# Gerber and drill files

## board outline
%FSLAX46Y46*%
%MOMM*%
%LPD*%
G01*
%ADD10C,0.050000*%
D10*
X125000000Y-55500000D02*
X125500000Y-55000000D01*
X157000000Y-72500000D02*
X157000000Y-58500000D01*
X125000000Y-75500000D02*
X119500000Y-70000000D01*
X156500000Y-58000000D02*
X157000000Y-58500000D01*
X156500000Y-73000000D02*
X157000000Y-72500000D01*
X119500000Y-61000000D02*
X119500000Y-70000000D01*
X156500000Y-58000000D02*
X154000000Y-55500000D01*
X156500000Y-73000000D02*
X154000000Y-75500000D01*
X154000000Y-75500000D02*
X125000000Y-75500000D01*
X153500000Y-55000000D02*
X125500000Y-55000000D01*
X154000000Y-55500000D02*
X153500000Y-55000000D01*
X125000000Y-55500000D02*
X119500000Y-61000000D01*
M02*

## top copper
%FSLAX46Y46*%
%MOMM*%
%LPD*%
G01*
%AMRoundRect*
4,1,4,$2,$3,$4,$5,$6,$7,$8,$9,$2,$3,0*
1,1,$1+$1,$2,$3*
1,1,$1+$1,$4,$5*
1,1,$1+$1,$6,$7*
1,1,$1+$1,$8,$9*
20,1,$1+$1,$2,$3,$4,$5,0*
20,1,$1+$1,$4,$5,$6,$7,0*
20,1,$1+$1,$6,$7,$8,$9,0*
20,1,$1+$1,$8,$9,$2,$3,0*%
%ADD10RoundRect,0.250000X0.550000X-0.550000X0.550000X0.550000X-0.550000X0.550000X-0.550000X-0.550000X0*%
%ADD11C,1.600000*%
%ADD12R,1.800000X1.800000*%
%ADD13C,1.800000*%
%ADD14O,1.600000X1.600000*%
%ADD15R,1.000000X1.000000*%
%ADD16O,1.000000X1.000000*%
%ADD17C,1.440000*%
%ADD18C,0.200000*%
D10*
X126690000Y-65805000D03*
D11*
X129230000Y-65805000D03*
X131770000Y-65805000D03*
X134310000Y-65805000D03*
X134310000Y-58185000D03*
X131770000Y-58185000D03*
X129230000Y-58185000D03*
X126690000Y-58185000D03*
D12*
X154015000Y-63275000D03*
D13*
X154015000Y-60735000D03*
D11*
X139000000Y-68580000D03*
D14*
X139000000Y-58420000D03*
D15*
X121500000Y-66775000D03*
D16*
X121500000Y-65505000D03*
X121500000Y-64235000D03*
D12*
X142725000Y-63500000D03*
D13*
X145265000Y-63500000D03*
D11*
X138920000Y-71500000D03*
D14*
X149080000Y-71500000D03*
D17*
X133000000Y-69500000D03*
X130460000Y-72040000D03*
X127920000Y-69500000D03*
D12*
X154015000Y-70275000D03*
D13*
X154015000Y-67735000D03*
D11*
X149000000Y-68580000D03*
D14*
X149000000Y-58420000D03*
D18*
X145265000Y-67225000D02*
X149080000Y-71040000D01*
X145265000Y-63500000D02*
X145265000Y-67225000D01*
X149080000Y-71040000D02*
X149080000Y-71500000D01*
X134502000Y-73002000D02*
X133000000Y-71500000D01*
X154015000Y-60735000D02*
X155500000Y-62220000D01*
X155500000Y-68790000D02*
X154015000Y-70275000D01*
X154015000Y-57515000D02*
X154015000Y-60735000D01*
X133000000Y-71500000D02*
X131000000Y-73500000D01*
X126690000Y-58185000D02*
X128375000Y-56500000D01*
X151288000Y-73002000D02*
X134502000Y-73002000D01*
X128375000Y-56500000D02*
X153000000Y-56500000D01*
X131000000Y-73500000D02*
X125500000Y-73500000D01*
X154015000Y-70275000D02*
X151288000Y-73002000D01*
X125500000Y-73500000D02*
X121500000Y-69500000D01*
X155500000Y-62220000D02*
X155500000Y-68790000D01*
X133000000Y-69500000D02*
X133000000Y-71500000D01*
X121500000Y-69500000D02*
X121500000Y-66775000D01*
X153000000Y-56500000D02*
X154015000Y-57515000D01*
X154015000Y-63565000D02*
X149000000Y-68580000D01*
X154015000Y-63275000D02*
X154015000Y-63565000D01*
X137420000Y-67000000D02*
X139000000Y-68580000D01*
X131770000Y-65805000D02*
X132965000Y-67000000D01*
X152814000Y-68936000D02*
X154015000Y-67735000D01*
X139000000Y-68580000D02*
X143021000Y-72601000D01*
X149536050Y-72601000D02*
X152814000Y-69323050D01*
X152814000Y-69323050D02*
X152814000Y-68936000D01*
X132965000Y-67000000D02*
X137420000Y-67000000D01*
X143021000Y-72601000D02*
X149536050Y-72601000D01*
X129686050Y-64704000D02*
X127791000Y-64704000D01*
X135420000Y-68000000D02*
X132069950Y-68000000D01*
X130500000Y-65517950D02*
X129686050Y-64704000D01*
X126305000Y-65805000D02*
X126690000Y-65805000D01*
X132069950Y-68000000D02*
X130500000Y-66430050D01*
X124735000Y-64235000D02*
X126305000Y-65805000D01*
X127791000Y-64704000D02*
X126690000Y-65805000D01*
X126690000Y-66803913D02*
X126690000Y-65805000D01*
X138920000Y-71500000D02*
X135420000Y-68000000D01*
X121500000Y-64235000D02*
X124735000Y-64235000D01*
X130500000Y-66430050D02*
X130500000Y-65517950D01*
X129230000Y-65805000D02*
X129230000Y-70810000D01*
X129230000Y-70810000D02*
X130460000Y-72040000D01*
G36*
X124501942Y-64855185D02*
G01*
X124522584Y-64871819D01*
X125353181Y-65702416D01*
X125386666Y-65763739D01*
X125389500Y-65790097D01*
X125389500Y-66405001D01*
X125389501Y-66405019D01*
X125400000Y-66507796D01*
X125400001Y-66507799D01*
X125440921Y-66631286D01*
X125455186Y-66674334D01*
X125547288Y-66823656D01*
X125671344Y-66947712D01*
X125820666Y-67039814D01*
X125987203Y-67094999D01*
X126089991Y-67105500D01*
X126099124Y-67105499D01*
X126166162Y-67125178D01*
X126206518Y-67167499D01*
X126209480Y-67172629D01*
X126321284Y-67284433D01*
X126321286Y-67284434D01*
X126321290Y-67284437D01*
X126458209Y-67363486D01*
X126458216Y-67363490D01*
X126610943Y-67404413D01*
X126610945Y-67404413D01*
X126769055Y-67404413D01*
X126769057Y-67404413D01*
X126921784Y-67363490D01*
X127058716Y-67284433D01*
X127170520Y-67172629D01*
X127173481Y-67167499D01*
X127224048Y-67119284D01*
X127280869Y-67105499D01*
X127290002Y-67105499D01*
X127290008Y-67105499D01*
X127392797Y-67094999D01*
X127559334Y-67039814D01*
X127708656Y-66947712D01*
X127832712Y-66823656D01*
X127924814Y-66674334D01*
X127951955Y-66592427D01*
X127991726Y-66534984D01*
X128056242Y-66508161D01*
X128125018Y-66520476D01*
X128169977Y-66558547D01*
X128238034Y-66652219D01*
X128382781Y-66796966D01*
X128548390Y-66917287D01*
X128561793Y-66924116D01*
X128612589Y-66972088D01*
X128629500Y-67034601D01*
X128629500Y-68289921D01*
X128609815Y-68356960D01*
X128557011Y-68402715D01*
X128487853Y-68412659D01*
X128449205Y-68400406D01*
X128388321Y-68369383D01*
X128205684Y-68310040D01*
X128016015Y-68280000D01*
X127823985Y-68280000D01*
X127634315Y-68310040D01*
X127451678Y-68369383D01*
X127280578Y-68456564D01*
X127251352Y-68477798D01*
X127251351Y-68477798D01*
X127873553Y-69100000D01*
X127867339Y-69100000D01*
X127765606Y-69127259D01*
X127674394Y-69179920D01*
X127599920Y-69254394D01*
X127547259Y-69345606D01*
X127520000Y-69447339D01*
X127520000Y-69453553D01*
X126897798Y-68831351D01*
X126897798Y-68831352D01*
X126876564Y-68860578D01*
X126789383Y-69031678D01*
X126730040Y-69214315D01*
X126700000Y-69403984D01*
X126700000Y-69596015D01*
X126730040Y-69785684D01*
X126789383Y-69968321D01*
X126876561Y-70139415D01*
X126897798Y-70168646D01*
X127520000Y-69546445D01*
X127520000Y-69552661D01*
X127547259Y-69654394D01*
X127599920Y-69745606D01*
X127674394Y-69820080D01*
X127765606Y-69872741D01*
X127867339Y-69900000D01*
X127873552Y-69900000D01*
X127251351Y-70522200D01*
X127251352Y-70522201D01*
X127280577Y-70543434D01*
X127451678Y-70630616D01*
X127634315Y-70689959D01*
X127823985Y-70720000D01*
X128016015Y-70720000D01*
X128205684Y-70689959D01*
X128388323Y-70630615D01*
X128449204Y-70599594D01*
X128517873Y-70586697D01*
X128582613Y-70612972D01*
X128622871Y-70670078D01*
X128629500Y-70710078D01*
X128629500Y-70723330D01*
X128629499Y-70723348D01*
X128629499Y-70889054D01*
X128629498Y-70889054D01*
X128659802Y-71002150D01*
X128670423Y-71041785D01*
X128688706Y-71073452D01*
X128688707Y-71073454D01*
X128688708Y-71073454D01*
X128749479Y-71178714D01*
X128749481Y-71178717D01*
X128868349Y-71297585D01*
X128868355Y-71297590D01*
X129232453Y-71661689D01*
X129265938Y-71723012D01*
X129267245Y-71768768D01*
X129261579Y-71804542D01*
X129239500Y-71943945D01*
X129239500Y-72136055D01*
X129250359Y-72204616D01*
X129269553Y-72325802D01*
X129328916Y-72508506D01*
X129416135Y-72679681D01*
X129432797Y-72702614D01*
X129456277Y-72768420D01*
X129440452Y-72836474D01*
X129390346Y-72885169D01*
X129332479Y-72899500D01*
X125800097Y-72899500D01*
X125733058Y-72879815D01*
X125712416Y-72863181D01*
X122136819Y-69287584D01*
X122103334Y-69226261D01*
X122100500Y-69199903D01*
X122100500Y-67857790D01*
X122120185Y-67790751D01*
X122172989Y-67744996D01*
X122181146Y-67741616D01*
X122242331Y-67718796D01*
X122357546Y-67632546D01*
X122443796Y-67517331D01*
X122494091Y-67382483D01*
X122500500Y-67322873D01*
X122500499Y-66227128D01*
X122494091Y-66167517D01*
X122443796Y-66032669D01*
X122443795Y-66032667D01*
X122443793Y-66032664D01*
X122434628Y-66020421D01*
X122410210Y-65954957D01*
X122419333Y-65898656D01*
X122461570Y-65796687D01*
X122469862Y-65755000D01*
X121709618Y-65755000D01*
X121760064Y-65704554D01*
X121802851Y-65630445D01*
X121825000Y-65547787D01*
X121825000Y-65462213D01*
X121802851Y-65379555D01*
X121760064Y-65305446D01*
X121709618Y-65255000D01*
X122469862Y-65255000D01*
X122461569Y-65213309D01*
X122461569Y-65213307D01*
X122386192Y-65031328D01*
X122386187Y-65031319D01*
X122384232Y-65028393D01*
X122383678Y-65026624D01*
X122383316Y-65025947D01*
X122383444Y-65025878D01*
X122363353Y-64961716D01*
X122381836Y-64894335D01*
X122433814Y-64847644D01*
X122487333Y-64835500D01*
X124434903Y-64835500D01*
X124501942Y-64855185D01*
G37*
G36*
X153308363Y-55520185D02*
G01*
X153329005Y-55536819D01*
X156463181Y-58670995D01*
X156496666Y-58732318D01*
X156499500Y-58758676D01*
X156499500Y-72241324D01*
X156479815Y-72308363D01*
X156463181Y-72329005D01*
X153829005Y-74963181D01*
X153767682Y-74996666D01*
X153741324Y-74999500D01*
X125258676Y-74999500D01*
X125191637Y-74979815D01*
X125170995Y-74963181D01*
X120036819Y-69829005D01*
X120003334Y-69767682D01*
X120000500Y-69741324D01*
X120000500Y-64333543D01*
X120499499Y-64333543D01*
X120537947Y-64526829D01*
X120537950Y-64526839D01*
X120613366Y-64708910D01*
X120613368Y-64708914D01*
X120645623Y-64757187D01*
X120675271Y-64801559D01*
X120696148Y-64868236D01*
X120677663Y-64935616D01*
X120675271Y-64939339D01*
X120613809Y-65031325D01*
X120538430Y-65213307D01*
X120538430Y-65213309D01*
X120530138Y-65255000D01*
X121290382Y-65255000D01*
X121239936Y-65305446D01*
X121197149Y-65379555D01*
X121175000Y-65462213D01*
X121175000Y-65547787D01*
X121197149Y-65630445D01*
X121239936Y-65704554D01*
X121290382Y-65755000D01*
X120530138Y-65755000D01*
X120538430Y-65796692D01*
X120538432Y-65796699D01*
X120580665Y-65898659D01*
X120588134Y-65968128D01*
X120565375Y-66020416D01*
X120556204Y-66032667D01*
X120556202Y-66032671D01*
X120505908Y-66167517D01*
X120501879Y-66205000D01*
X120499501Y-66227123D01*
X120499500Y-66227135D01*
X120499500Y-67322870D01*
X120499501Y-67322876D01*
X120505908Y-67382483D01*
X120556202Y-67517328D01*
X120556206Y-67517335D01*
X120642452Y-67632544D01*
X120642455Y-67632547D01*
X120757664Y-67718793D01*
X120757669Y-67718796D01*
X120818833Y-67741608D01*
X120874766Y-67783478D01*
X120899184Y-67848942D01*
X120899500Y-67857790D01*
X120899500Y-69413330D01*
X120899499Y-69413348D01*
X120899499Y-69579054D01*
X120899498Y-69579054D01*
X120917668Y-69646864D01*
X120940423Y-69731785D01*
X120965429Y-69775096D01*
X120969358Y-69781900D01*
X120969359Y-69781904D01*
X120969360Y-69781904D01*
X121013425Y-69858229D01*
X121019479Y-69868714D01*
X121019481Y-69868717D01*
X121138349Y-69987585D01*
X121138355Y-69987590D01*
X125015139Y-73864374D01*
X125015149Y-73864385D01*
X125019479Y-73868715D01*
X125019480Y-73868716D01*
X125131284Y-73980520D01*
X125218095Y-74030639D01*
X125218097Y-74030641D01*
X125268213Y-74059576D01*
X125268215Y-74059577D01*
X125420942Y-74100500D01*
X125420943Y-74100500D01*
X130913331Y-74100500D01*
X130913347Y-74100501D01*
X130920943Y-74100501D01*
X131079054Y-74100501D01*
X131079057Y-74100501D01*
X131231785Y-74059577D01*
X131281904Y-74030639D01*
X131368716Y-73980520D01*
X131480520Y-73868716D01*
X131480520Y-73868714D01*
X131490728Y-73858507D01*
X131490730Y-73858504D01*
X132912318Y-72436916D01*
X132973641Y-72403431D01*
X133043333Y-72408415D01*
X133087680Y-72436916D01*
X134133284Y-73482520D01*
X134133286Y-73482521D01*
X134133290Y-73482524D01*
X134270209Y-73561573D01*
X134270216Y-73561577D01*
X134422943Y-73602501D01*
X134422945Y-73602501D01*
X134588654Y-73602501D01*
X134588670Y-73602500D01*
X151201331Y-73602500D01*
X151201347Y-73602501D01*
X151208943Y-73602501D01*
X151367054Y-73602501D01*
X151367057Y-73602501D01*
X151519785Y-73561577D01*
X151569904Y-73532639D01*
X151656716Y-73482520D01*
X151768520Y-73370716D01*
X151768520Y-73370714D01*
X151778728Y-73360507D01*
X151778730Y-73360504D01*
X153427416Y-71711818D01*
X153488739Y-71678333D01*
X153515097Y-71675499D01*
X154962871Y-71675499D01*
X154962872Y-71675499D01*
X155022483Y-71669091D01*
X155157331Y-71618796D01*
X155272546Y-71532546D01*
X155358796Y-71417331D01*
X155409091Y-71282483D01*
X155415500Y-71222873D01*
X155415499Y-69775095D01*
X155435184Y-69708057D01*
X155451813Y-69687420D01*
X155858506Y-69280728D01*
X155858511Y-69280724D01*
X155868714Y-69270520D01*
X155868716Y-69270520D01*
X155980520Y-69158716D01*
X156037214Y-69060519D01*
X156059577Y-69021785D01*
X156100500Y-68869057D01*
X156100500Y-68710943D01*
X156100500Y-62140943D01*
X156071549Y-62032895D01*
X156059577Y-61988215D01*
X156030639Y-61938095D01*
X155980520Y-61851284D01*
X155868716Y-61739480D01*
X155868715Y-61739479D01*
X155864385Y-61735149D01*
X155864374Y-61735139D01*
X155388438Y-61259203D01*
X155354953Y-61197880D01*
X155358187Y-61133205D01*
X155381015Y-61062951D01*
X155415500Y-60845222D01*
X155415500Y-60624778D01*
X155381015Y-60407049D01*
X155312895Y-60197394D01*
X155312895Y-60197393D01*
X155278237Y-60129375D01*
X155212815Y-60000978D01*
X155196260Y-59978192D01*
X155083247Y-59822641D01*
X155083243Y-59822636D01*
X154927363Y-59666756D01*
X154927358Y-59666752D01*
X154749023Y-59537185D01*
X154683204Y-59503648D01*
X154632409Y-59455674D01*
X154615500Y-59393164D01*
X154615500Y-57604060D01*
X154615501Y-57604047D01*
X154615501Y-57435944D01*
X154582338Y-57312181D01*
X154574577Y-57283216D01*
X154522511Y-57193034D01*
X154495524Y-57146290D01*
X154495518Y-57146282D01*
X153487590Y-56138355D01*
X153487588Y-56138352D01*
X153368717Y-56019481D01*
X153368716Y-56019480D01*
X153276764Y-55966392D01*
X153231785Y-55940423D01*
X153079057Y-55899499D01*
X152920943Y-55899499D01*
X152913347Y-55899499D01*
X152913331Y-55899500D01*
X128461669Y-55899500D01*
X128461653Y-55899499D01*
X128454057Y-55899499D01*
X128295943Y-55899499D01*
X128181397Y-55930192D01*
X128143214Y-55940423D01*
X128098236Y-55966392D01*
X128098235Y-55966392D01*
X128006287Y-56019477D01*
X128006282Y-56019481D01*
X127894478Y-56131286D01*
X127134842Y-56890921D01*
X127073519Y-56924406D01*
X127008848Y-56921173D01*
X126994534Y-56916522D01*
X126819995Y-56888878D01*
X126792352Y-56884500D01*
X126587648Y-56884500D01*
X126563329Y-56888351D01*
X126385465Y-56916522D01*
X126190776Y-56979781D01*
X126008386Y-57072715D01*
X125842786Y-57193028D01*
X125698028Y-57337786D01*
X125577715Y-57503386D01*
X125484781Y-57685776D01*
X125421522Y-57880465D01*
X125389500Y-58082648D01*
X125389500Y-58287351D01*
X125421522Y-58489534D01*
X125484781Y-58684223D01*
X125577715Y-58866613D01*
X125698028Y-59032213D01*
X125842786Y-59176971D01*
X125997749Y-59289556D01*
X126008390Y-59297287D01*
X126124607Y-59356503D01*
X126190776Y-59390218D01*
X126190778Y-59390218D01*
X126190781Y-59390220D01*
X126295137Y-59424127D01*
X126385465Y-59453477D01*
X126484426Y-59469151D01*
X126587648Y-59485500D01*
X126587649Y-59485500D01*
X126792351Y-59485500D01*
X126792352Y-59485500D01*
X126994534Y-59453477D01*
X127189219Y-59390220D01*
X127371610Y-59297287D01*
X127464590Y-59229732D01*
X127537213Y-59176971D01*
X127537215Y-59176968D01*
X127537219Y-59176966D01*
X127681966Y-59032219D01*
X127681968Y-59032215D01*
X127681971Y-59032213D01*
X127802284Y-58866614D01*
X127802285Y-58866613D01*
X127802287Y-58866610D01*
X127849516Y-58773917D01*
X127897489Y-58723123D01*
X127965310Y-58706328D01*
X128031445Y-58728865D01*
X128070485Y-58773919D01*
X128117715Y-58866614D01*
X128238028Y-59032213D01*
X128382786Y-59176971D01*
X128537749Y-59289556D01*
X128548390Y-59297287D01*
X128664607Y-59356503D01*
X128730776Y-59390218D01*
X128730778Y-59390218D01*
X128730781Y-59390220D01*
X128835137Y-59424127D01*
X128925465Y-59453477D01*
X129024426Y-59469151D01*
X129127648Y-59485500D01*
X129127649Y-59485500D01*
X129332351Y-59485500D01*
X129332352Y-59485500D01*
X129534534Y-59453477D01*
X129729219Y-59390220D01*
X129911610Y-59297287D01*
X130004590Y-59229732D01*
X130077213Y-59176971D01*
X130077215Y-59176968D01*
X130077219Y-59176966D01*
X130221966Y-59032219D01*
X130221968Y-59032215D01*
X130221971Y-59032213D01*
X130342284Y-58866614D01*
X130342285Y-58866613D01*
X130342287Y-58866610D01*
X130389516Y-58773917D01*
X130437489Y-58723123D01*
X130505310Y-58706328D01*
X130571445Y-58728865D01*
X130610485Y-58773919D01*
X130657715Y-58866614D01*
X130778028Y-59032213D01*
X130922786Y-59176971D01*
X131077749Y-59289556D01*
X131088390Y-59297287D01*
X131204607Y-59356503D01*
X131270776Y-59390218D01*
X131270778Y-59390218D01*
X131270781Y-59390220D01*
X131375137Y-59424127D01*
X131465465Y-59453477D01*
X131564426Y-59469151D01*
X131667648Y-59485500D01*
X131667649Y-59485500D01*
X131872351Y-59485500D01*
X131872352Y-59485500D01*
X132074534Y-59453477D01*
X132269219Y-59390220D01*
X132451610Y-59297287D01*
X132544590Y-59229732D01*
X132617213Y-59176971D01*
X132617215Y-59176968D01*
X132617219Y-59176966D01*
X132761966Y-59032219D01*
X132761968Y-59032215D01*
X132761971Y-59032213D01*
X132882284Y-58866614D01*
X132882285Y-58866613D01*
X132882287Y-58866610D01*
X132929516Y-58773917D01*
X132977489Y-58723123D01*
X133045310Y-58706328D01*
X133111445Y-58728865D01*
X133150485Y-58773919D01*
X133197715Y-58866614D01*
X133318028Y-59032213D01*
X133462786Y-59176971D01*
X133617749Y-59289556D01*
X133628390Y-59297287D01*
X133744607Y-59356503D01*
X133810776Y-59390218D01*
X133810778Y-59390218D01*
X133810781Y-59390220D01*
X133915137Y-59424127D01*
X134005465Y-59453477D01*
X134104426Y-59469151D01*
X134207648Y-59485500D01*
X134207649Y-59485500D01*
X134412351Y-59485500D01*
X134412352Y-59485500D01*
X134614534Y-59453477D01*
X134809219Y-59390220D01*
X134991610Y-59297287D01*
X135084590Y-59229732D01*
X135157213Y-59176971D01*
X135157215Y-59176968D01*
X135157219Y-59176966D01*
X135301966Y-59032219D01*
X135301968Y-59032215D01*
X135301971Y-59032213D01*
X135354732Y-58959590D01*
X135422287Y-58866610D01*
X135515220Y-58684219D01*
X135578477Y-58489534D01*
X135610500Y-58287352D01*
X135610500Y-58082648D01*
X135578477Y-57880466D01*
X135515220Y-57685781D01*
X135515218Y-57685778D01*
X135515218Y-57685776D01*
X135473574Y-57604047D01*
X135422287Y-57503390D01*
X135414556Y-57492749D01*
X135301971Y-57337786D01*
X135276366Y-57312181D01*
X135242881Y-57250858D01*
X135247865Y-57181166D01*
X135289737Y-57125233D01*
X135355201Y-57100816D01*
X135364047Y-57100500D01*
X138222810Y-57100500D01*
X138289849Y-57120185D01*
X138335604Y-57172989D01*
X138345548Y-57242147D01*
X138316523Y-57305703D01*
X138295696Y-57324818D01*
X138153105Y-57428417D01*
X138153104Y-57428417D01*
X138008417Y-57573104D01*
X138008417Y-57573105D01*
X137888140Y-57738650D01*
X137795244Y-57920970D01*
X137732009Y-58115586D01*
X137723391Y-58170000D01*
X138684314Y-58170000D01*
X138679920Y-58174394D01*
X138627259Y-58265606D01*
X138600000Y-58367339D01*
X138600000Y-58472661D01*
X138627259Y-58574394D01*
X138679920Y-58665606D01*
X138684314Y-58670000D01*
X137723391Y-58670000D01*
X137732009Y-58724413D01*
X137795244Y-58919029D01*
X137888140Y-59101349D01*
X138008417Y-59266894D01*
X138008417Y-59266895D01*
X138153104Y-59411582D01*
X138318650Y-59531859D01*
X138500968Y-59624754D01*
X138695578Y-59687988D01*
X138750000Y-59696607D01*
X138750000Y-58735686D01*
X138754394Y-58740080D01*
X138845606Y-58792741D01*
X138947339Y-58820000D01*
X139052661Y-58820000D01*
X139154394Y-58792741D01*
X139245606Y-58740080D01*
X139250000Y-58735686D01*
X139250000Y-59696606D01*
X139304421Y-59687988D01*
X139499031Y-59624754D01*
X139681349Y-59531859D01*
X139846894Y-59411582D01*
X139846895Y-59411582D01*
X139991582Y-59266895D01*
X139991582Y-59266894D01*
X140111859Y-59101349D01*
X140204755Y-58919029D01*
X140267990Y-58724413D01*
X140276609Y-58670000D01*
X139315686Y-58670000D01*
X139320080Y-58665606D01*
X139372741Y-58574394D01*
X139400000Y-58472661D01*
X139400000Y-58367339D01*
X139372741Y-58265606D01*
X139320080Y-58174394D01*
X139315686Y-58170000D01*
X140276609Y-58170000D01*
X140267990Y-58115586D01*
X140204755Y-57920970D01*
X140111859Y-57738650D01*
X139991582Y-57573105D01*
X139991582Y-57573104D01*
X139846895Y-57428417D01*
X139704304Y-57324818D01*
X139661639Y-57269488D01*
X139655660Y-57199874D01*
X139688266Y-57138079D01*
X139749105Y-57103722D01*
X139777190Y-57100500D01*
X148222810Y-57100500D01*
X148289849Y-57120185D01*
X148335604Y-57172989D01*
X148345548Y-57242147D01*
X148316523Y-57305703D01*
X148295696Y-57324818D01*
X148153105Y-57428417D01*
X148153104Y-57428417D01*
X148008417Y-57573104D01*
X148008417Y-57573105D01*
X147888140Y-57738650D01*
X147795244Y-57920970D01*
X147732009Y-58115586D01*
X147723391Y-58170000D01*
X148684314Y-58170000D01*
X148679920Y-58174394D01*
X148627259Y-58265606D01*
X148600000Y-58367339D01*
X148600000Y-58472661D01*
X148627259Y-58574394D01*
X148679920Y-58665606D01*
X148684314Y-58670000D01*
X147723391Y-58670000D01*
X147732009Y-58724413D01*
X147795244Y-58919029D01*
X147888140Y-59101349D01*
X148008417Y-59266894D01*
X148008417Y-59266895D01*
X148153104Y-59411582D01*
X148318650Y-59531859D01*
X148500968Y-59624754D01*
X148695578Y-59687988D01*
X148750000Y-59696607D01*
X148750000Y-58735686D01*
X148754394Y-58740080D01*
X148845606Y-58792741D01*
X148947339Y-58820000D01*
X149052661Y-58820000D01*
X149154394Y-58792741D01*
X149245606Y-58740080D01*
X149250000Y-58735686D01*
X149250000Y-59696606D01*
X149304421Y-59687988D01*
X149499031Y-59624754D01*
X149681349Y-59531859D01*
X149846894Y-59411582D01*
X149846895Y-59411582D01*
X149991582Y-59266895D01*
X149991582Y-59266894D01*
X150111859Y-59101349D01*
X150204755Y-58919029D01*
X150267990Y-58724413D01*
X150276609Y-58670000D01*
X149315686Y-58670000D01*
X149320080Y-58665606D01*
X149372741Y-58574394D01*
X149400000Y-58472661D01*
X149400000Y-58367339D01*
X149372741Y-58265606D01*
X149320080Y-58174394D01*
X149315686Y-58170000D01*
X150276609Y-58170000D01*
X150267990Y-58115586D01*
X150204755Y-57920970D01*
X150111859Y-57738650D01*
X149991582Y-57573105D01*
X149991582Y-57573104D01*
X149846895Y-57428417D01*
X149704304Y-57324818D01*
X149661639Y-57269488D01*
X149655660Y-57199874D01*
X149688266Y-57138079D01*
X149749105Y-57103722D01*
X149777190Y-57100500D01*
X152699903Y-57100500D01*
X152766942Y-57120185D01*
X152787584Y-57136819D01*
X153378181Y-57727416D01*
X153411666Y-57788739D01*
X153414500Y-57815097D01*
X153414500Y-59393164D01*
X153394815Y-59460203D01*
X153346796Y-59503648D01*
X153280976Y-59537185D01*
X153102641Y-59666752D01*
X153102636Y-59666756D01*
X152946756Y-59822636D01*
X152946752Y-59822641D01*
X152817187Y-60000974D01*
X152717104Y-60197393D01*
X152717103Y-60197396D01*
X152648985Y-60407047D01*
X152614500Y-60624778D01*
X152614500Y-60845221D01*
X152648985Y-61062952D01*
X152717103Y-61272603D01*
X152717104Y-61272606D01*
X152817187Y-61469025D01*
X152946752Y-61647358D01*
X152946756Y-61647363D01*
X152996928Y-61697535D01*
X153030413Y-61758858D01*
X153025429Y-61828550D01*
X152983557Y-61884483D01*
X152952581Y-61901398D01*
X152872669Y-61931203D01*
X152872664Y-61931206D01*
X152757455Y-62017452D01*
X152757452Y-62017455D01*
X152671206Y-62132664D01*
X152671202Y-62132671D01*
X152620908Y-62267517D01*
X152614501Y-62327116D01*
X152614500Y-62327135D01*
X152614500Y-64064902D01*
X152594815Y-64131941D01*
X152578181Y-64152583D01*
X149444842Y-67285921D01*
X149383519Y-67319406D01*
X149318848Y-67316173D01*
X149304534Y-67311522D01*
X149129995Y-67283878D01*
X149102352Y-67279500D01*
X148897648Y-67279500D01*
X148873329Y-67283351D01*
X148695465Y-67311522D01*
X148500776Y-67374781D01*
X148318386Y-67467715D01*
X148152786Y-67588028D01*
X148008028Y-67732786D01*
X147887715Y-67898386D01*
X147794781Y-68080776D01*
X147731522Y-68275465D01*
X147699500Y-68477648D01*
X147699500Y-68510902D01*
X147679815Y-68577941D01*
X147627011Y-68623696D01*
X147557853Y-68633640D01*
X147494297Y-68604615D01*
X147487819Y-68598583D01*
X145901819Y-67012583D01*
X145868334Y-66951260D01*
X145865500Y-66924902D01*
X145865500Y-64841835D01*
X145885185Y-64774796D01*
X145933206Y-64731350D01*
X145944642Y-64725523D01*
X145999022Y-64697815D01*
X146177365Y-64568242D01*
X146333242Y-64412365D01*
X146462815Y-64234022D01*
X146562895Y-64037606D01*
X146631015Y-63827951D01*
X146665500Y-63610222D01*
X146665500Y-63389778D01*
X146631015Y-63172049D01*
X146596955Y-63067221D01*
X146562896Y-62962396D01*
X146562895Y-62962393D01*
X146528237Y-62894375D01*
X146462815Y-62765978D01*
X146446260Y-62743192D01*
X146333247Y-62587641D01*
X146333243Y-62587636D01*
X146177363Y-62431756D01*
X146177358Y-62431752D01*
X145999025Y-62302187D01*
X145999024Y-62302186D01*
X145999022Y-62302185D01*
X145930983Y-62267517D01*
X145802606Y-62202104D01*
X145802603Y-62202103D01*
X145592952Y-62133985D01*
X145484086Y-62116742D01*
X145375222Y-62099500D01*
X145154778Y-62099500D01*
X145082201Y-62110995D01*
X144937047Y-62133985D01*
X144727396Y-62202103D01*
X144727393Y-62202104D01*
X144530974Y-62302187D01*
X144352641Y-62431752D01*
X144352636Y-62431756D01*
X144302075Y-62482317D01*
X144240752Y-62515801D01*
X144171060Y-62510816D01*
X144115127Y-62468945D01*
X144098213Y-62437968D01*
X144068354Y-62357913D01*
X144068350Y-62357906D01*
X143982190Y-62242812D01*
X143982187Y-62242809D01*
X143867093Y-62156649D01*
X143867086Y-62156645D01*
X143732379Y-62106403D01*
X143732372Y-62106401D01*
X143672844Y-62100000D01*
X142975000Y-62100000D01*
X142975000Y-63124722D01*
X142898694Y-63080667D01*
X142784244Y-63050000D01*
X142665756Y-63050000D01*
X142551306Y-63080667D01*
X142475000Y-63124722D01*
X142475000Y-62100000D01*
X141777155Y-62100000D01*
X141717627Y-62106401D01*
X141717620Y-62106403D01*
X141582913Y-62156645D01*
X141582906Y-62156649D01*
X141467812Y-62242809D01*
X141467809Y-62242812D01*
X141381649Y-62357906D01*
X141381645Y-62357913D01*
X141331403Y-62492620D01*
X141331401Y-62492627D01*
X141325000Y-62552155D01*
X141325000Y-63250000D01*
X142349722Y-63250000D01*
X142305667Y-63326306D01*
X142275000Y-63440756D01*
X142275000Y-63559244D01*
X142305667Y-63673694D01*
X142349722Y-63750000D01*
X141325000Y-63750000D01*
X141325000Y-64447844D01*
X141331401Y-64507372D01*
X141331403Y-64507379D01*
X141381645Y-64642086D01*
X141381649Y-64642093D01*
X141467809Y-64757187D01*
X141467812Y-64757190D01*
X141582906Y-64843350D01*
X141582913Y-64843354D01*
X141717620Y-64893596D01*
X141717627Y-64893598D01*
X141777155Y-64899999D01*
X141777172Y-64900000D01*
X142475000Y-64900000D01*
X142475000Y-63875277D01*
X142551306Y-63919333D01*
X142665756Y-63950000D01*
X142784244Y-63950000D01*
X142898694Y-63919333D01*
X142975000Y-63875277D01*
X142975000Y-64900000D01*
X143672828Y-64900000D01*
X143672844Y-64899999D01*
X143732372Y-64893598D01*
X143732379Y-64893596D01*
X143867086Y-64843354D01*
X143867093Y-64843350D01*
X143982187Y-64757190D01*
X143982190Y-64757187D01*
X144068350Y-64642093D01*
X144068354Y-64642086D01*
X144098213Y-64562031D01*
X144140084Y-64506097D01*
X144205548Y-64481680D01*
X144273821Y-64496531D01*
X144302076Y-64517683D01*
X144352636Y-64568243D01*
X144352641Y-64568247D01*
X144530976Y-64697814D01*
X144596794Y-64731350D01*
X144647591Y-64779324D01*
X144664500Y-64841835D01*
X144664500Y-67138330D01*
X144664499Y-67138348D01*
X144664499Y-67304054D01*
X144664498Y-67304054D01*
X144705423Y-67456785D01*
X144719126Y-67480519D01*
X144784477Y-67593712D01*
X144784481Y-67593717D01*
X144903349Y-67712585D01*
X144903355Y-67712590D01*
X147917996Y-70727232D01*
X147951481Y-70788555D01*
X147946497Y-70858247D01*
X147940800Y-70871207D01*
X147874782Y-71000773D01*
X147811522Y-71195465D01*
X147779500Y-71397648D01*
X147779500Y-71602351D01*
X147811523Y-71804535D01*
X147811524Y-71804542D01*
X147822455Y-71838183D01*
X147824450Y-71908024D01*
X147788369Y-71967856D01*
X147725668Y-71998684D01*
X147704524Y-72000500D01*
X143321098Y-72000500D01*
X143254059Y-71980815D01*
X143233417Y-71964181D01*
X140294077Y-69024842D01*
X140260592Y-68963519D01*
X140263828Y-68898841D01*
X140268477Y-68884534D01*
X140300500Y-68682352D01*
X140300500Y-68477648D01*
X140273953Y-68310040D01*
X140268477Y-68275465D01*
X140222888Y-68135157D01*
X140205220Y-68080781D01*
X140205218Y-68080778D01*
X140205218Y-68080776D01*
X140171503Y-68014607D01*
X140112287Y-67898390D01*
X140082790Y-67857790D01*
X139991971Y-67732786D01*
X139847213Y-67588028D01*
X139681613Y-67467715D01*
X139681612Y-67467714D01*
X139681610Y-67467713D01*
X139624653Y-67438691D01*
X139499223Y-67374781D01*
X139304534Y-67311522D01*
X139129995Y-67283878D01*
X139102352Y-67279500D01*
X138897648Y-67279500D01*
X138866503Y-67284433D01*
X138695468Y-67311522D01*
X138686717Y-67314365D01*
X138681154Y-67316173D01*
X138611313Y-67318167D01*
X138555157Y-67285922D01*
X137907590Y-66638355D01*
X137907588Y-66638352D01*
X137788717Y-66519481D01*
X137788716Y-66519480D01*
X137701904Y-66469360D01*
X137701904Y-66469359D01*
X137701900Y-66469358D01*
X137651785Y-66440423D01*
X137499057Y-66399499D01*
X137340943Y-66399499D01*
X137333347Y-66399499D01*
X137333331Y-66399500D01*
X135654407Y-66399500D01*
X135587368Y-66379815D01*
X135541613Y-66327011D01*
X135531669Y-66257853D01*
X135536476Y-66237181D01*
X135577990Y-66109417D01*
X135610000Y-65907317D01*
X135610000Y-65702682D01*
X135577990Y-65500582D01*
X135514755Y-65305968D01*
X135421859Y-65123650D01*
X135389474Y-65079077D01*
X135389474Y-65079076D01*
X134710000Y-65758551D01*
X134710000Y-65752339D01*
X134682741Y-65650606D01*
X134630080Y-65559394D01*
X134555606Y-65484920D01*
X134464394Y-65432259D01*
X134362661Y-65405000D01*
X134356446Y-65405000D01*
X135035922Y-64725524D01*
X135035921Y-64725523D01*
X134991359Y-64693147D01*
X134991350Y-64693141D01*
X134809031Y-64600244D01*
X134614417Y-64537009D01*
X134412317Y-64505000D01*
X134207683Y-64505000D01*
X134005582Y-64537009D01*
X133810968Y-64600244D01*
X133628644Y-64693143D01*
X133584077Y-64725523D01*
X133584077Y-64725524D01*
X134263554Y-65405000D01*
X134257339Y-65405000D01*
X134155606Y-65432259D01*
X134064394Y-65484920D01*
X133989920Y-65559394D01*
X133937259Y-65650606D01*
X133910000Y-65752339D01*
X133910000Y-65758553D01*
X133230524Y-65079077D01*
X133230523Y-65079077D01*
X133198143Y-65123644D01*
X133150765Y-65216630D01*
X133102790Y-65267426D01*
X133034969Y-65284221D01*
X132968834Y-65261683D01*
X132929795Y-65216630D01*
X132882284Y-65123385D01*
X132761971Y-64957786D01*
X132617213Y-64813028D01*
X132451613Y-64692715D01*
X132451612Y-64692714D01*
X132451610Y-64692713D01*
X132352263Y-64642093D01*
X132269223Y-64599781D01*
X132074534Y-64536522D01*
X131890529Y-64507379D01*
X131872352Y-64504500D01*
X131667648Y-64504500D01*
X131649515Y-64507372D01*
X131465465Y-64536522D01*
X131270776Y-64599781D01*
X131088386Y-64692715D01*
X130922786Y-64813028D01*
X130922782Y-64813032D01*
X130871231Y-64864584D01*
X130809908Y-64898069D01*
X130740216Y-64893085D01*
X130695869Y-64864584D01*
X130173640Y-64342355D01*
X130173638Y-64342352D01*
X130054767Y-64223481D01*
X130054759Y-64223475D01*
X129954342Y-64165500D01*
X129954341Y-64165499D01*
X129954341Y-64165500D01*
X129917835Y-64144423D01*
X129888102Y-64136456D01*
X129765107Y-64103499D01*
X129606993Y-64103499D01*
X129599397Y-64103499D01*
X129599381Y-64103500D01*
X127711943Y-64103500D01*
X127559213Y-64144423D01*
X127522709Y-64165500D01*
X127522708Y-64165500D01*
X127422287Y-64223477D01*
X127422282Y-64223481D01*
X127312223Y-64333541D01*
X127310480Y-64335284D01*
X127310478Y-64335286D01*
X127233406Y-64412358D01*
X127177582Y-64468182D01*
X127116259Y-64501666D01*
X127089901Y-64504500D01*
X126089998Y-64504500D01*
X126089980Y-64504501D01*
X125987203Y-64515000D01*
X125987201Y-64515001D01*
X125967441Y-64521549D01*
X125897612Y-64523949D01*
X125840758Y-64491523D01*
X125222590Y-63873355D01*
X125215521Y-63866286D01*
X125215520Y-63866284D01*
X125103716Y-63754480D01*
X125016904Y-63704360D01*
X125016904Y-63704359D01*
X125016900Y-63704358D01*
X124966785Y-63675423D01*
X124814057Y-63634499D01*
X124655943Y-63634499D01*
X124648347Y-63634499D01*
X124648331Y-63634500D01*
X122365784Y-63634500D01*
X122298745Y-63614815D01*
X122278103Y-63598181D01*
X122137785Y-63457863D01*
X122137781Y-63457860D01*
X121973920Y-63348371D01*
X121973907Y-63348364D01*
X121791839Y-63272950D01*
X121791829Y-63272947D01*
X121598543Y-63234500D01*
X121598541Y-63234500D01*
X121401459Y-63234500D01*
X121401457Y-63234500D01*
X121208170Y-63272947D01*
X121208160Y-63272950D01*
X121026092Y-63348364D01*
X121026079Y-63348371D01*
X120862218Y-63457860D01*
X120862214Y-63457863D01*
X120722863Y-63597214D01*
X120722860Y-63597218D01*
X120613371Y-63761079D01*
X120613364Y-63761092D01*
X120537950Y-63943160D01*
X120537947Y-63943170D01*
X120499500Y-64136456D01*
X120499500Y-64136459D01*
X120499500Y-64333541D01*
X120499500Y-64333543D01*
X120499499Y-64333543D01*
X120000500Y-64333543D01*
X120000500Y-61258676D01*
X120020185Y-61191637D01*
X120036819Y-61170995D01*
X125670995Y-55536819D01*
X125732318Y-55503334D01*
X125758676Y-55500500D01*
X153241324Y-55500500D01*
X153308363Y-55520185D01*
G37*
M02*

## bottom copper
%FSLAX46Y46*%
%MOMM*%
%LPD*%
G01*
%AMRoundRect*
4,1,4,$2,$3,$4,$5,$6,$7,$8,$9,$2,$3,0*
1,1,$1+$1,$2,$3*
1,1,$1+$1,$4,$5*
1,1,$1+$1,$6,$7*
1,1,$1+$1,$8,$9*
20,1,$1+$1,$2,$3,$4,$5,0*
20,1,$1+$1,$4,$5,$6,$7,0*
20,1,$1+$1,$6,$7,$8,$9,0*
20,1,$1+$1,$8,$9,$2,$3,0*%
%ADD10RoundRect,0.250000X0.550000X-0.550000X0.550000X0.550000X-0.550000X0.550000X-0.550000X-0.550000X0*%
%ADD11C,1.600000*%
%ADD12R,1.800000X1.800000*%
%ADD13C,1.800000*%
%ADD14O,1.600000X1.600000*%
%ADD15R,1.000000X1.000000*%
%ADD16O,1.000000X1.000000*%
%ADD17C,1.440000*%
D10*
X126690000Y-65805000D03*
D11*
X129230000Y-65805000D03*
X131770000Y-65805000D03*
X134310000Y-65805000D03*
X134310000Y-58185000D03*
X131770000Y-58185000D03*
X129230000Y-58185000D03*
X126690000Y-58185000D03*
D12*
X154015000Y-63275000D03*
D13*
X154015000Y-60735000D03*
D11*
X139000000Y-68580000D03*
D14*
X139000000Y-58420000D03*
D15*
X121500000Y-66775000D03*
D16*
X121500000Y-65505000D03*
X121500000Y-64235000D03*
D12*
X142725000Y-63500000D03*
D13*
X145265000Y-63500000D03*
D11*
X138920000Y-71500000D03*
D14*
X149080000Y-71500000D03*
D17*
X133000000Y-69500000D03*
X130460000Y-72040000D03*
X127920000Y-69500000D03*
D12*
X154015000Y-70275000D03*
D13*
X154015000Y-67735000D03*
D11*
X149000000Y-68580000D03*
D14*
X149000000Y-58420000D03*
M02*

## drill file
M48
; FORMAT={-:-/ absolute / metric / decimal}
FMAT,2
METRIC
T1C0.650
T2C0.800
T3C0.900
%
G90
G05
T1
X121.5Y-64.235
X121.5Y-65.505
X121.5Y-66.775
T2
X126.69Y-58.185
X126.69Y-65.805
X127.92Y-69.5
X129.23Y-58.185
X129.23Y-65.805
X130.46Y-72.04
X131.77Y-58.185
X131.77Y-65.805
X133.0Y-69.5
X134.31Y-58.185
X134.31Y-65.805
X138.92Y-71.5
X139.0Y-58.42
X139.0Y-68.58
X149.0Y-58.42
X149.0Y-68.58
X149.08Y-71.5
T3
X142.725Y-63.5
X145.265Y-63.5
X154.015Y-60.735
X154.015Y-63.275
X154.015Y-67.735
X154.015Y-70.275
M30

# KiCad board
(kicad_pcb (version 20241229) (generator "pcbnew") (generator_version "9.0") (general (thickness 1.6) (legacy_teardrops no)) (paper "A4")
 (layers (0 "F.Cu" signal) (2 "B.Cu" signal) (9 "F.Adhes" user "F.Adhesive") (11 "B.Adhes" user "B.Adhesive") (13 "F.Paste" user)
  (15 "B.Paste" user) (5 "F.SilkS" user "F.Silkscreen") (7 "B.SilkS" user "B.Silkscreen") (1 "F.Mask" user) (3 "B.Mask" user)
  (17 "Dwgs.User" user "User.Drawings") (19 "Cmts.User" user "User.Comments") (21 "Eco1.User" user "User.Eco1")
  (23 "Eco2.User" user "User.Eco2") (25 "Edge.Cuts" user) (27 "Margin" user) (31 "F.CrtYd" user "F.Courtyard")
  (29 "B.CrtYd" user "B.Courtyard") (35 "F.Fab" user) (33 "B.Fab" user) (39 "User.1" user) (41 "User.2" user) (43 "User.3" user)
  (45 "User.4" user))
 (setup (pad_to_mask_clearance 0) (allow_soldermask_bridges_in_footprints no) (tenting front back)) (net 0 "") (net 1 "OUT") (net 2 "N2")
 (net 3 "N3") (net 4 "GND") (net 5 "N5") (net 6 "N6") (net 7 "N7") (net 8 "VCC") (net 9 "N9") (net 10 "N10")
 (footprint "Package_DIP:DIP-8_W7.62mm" (layer "F.Cu") (at 126.69 65.805 90)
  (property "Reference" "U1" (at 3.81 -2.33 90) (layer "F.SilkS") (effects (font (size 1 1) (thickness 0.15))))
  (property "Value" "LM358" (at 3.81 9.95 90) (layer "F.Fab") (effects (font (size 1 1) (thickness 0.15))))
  (pad "1" thru_hole roundrect (at 0 0 90) (size 1.6 1.6) (drill 0.8) (layers "*.Cu" "*.Mask") (remove_unused_layers no)
   (roundrect_rratio 0.15625) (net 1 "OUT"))
  (pad "2" thru_hole circle (at 0 2.54 90) (size 1.6 1.6) (drill 0.8) (layers "*.Cu" "*.Mask") (remove_unused_layers no) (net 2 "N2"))
  (pad "3" thru_hole circle (at 0 5.08 90) (size 1.6 1.6) (drill 0.8) (layers "*.Cu" "*.Mask") (remove_unused_layers no) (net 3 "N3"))
  (pad "4" thru_hole circle (at 0 7.62 90) (size 1.6 1.6) (drill 0.8) (layers "*.Cu" "*.Mask") (remove_unused_layers no) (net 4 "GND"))
  (pad "5" thru_hole circle (at 7.62 7.62 90) (size 1.6 1.6) (drill 0.8) (layers "*.Cu" "*.Mask") (remove_unused_layers no) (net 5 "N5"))
  (pad "6" thru_hole circle (at 7.62 5.08 90) (size 1.6 1.6) (drill 0.8) (layers "*.Cu" "*.Mask") (remove_unused_layers no) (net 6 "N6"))
  (pad "7" thru_hole circle (at 7.62 2.54 90) (size 1.6 1.6) (drill 0.8) (layers "*.Cu" "*.Mask") (remove_unused_layers no) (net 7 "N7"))
  (pad "8" thru_hole circle (at 7.62 0 90) (size 1.6 1.6) (drill 0.8) (layers "*.Cu" "*.Mask") (remove_unused_layers no) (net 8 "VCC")))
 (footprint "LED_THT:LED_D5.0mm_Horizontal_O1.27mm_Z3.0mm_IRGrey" (layer "F.Cu") (at 154.015 63.275 90)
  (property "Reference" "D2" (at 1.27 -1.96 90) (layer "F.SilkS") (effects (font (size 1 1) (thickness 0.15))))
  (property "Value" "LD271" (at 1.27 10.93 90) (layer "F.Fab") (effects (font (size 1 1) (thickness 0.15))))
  (pad "1" thru_hole rect (at 0 0 90) (size 1.8 1.8) (drill 0.9) (layers "*.Cu" "*.Mask") (remove_unused_layers no) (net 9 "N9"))
  (pad "2" thru_hole circle (at 2.54 0 90) (size 1.8 1.8) (drill 0.9) (layers "*.Cu" "*.Mask") (remove_unused_layers no) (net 8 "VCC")))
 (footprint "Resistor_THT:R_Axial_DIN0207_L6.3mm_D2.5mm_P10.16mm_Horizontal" (layer "F.Cu") (at 139 68.58 90)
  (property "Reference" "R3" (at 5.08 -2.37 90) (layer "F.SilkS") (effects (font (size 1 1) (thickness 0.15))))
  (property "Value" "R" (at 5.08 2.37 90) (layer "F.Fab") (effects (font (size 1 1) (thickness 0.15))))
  (pad "1" thru_hole circle (at 0 0 90) (size 1.6 1.6) (drill 0.8) (layers "*.Cu" "*.Mask") (remove_unused_layers no) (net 3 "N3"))
  (pad "2" thru_hole oval (at 10.16 0 90) (size 1.6 1.6) (drill 0.8) (layers "*.Cu" "*.Mask") (remove_unused_layers no) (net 4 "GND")))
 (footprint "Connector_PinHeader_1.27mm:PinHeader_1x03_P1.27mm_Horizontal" (layer "F.Cu") (at 121.5 66.775 180)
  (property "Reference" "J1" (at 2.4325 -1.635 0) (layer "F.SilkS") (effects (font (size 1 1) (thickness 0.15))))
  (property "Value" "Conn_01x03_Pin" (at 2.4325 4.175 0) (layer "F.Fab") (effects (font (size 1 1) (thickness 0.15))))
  (pad "1" thru_hole rect (at 0 0 180) (size 1 1) (drill 0.65) (layers "*.Cu" "*.Mask") (remove_unused_layers no) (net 8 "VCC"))
  (pad "2" thru_hole oval (at 0 1.27 180) (size 1 1) (drill 0.65) (layers "*.Cu" "*.Mask") (remove_unused_layers no) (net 4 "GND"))
  (pad "3" thru_hole oval (at 0 2.54 180) (size 1 1) (drill 0.65) (layers "*.Cu" "*.Mask") (remove_unused_layers no) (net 1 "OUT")))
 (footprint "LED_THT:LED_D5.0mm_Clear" (layer "F.Cu") (at 142.725 63.5)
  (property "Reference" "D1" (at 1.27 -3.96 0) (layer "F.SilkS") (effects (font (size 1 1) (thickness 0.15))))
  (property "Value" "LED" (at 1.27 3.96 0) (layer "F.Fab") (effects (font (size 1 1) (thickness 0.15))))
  (pad "1" thru_hole rect (at 0 0) (size 1.8 1.8) (drill 0.9) (layers "*.Cu" "*.Mask") (remove_unused_layers no) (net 4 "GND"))
  (pad "2" thru_hole circle (at 2.54 0) (size 1.8 1.8) (drill 0.9) (layers "*.Cu" "*.Mask") (remove_unused_layers no) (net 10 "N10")))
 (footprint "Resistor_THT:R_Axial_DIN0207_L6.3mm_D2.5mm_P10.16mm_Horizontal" (layer "F.Cu") (at 138.92 71.5)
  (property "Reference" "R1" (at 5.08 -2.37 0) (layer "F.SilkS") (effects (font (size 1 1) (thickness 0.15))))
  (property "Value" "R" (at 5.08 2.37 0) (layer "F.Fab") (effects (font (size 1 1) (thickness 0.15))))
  (pad "1" thru_hole circle (at 0 0) (size 1.6 1.6) (drill 0.8) (layers "*.Cu" "*.Mask") (remove_unused_layers no) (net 1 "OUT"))
  (pad "2" thru_hole oval (at 10.16 0) (size 1.6 1.6) (drill 0.8) (layers "*.Cu" "*.Mask") (remove_unused_layers no) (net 10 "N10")))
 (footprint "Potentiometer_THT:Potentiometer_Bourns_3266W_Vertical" (layer "F.Cu") (at 133 69.5)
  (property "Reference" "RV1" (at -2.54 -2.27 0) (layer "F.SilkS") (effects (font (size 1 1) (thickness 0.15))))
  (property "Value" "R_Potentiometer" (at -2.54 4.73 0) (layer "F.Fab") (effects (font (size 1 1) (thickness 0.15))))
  (pad "1" thru_hole circle (at 0 0) (size 1.44 1.44) (drill 0.8) (layers "*.Cu" "*.Mask") (remove_unused_layers no) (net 8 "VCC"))
  (pad "2" thru_hole circle (at -2.54 2.54) (size 1.44 1.44) (drill 0.8) (layers "*.Cu" "*.Mask") (remove_unused_layers no) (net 2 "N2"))
  (pad "3" thru_hole circle (at -5.08 0) (size 1.44 1.44) (drill 0.8) (layers "*.Cu" "*.Mask") (remove_unused_layers no) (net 4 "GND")))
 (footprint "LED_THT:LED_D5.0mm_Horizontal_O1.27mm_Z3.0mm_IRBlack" (layer "F.Cu") (at 154.015 70.275 90)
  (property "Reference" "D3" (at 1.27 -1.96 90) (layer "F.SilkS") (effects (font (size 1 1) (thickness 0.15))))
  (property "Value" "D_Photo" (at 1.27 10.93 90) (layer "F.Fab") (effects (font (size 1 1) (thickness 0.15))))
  (pad "1" thru_hole rect (at 0 0 90) (size 1.8 1.8) (drill 0.9) (layers "*.Cu" "*.Mask") (remove_unused_layers no) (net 8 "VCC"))
  (pad "2" thru_hole circle (at 2.54 0 90) (size 1.8 1.8) (drill 0.9) (layers "*.Cu" "*.Mask") (remove_unused_layers no) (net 3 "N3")))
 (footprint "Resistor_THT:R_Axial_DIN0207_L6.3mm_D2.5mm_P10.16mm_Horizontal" (layer "F.Cu") (at 149 68.58 90)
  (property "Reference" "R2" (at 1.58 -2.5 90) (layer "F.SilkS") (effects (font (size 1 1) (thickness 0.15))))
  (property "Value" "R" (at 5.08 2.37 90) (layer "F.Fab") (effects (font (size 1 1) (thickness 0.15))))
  (pad "1" thru_hole circle (at 0 0 90) (size 1.6 1.6) (drill 0.8) (layers "*.Cu" "*.Mask") (remove_unused_layers no) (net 9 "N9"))
  (pad "2" thru_hole oval (at 10.16 0 90) (size 1.6 1.6) (drill 0.8) (layers "*.Cu" "*.Mask") (remove_unused_layers no) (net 4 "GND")))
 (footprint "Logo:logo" (layer "B.Cu") (at 140.5 70.5 180)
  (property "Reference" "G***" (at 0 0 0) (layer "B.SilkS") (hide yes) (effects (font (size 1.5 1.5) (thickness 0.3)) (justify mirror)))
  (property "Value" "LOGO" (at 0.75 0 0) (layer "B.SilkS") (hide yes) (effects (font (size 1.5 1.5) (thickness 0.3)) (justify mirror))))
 (gr_line (start 125 55.5) (end 125.5 55) (stroke (width 0.05) (type default)) (layer "Edge.Cuts"))
 (gr_line (start 157 72.5) (end 157 58.5) (stroke (width 0.05) (type default)) (layer "Edge.Cuts"))
 (gr_line (start 125 75.5) (end 119.5 70) (stroke (width 0.05) (type default)) (layer "Edge.Cuts"))
 (gr_line (start 156.5 58) (end 157 58.5) (stroke (width 0.05) (type default)) (layer "Edge.Cuts"))
 (gr_line (start 156.5 73) (end 157 72.5) (stroke (width 0.05) (type default)) (layer "Edge.Cuts"))
 (gr_line (start 119.5 61) (end 119.5 70) (stroke (width 0.05) (type default)) (layer "Edge.Cuts"))
 (gr_line (start 156.5 58) (end 154 55.5) (stroke (width 0.05) (type default)) (layer "Edge.Cuts"))
 (gr_line (start 156.5 73) (end 154 75.5) (stroke (width 0.05) (type default)) (layer "Edge.Cuts"))
 (gr_line (start 154 75.5) (end 125 75.5) (stroke (width 0.05) (type default)) (layer "Edge.Cuts"))
 (gr_line (start 153.5 55) (end 125.5 55) (stroke (width 0.05) (type default)) (layer "Edge.Cuts"))
 (gr_line (start 154 55.5) (end 153.5 55) (stroke (width 0.05) (type default)) (layer "Edge.Cuts"))
 (gr_line (start 125 55.5) (end 119.5 61) (stroke (width 0.05) (type default)) (layer "Edge.Cuts"))
 (segment (start 145.265 67.225) (end 149.08 71.04) (width 0.2) (layer "F.Cu") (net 10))
 (segment (start 145.265 63.5) (end 145.265 67.225) (width 0.2) (layer "F.Cu") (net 10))
 (segment (start 149.08 71.04) (end 149.08 71.5) (width 0.2) (layer "F.Cu") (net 10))
 (segment (start 134.502 73.002) (end 133 71.5) (width 0.2) (layer "F.Cu") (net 8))
 (segment (start 154.015 60.735) (end 155.5 62.22) (width 0.2) (layer "F.Cu") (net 8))
 (segment (start 155.5 68.79) (end 154.015 70.275) (width 0.2) (layer "F.Cu") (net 8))
 (segment (start 154.015 57.515) (end 154.015 60.735) (width 0.2) (layer "F.Cu") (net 8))
 (segment (start 133 71.5) (end 131 73.5) (width 0.2) (layer "F.Cu") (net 8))
 (segment (start 126.69 58.185) (end 128.375 56.5) (width 0.2) (layer "F.Cu") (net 8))
 (segment (start 151.288 73.002) (end 134.502 73.002) (width 0.2) (layer "F.Cu") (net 8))
 (segment (start 128.375 56.5) (end 153 56.5) (width 0.2) (layer "F.Cu") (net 8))
 (segment (start 131 73.5) (end 125.5 73.5) (width 0.2) (layer "F.Cu") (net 8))
 (segment (start 154.015 70.275) (end 151.288 73.002) (width 0.2) (layer "F.Cu") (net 8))
 (segment (start 125.5 73.5) (end 121.5 69.5) (width 0.2) (layer "F.Cu") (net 8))
 (segment (start 155.5 62.22) (end 155.5 68.79) (width 0.2) (layer "F.Cu") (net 8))
 (segment (start 133 69.5) (end 133 71.5) (width 0.2) (layer "F.Cu") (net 8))
 (segment (start 121.5 69.5) (end 121.5 66.775) (width 0.2) (layer "F.Cu") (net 8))
 (segment (start 153 56.5) (end 154.015 57.515) (width 0.2) (layer "F.Cu") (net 8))
 (segment (start 154.015 63.565) (end 149 68.58) (width 0.2) (layer "F.Cu") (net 9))
 (segment (start 154.015 63.275) (end 154.015 63.565) (width 0.2) (layer "F.Cu") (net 9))
 (segment (start 137.42 67) (end 139 68.58) (width 0.2) (layer "F.Cu") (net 3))
 (segment (start 131.77 65.805) (end 132.965 67) (width 0.2) (layer "F.Cu") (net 3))
 (segment (start 152.814 68.936) (end 154.015 67.735) (width 0.2) (layer "F.Cu") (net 3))
 (segment (start 139 68.58) (end 143.021 72.601) (width 0.2) (layer "F.Cu") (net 3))
 (segment (start 149.53605 72.601) (end 152.814 69.32305) (width 0.2) (layer "F.Cu") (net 3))
 (segment (start 152.814 69.32305) (end 152.814 68.936) (width 0.2) (layer "F.Cu") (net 3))
 (segment (start 132.965 67) (end 137.42 67) (width 0.2) (layer "F.Cu") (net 3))
 (segment (start 143.021 72.601) (end 149.53605 72.601) (width 0.2) (layer "F.Cu") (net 3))
 (segment (start 129.68605 64.704) (end 127.791 64.704) (width 0.2) (layer "F.Cu") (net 1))
 (segment (start 135.42 68) (end 132.06995 68) (width 0.2) (layer "F.Cu") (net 1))
 (segment (start 130.5 65.51795) (end 129.68605 64.704) (width 0.2) (layer "F.Cu") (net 1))
 (segment (start 126.305 65.805) (end 126.69 65.805) (width 0.2) (layer "F.Cu") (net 1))
 (segment (start 132.06995 68) (end 130.5 66.43005) (width 0.2) (layer "F.Cu") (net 1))
 (segment (start 124.735 64.235) (end 126.305 65.805) (width 0.2) (layer "F.Cu") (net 1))
 (segment (start 127.791 64.704) (end 126.69 65.805) (width 0.2) (layer "F.Cu") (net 1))
 (segment (start 126.69 66.803913) (end 126.69 65.805) (width 0.2) (layer "F.Cu") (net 1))
 (segment (start 138.92 71.5) (end 135.42 68) (width 0.2) (layer "F.Cu") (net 1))
 (segment (start 121.5 64.235) (end 124.735 64.235) (width 0.2) (layer "F.Cu") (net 1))
 (segment (start 130.5 66.43005) (end 130.5 65.51795) (width 0.2) (layer "F.Cu") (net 1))
 (segment (start 129.23 65.805) (end 129.23 70.81) (width 0.2) (layer "F.Cu") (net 2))
 (segment (start 129.23 70.81) (end 130.46 72.04) (width 0.2) (layer "F.Cu") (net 2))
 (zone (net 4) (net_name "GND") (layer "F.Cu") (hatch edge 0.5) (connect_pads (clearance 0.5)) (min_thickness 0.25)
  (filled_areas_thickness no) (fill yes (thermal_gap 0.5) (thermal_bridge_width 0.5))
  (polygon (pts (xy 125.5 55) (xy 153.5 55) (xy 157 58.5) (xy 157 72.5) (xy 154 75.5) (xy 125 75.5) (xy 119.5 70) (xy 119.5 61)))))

